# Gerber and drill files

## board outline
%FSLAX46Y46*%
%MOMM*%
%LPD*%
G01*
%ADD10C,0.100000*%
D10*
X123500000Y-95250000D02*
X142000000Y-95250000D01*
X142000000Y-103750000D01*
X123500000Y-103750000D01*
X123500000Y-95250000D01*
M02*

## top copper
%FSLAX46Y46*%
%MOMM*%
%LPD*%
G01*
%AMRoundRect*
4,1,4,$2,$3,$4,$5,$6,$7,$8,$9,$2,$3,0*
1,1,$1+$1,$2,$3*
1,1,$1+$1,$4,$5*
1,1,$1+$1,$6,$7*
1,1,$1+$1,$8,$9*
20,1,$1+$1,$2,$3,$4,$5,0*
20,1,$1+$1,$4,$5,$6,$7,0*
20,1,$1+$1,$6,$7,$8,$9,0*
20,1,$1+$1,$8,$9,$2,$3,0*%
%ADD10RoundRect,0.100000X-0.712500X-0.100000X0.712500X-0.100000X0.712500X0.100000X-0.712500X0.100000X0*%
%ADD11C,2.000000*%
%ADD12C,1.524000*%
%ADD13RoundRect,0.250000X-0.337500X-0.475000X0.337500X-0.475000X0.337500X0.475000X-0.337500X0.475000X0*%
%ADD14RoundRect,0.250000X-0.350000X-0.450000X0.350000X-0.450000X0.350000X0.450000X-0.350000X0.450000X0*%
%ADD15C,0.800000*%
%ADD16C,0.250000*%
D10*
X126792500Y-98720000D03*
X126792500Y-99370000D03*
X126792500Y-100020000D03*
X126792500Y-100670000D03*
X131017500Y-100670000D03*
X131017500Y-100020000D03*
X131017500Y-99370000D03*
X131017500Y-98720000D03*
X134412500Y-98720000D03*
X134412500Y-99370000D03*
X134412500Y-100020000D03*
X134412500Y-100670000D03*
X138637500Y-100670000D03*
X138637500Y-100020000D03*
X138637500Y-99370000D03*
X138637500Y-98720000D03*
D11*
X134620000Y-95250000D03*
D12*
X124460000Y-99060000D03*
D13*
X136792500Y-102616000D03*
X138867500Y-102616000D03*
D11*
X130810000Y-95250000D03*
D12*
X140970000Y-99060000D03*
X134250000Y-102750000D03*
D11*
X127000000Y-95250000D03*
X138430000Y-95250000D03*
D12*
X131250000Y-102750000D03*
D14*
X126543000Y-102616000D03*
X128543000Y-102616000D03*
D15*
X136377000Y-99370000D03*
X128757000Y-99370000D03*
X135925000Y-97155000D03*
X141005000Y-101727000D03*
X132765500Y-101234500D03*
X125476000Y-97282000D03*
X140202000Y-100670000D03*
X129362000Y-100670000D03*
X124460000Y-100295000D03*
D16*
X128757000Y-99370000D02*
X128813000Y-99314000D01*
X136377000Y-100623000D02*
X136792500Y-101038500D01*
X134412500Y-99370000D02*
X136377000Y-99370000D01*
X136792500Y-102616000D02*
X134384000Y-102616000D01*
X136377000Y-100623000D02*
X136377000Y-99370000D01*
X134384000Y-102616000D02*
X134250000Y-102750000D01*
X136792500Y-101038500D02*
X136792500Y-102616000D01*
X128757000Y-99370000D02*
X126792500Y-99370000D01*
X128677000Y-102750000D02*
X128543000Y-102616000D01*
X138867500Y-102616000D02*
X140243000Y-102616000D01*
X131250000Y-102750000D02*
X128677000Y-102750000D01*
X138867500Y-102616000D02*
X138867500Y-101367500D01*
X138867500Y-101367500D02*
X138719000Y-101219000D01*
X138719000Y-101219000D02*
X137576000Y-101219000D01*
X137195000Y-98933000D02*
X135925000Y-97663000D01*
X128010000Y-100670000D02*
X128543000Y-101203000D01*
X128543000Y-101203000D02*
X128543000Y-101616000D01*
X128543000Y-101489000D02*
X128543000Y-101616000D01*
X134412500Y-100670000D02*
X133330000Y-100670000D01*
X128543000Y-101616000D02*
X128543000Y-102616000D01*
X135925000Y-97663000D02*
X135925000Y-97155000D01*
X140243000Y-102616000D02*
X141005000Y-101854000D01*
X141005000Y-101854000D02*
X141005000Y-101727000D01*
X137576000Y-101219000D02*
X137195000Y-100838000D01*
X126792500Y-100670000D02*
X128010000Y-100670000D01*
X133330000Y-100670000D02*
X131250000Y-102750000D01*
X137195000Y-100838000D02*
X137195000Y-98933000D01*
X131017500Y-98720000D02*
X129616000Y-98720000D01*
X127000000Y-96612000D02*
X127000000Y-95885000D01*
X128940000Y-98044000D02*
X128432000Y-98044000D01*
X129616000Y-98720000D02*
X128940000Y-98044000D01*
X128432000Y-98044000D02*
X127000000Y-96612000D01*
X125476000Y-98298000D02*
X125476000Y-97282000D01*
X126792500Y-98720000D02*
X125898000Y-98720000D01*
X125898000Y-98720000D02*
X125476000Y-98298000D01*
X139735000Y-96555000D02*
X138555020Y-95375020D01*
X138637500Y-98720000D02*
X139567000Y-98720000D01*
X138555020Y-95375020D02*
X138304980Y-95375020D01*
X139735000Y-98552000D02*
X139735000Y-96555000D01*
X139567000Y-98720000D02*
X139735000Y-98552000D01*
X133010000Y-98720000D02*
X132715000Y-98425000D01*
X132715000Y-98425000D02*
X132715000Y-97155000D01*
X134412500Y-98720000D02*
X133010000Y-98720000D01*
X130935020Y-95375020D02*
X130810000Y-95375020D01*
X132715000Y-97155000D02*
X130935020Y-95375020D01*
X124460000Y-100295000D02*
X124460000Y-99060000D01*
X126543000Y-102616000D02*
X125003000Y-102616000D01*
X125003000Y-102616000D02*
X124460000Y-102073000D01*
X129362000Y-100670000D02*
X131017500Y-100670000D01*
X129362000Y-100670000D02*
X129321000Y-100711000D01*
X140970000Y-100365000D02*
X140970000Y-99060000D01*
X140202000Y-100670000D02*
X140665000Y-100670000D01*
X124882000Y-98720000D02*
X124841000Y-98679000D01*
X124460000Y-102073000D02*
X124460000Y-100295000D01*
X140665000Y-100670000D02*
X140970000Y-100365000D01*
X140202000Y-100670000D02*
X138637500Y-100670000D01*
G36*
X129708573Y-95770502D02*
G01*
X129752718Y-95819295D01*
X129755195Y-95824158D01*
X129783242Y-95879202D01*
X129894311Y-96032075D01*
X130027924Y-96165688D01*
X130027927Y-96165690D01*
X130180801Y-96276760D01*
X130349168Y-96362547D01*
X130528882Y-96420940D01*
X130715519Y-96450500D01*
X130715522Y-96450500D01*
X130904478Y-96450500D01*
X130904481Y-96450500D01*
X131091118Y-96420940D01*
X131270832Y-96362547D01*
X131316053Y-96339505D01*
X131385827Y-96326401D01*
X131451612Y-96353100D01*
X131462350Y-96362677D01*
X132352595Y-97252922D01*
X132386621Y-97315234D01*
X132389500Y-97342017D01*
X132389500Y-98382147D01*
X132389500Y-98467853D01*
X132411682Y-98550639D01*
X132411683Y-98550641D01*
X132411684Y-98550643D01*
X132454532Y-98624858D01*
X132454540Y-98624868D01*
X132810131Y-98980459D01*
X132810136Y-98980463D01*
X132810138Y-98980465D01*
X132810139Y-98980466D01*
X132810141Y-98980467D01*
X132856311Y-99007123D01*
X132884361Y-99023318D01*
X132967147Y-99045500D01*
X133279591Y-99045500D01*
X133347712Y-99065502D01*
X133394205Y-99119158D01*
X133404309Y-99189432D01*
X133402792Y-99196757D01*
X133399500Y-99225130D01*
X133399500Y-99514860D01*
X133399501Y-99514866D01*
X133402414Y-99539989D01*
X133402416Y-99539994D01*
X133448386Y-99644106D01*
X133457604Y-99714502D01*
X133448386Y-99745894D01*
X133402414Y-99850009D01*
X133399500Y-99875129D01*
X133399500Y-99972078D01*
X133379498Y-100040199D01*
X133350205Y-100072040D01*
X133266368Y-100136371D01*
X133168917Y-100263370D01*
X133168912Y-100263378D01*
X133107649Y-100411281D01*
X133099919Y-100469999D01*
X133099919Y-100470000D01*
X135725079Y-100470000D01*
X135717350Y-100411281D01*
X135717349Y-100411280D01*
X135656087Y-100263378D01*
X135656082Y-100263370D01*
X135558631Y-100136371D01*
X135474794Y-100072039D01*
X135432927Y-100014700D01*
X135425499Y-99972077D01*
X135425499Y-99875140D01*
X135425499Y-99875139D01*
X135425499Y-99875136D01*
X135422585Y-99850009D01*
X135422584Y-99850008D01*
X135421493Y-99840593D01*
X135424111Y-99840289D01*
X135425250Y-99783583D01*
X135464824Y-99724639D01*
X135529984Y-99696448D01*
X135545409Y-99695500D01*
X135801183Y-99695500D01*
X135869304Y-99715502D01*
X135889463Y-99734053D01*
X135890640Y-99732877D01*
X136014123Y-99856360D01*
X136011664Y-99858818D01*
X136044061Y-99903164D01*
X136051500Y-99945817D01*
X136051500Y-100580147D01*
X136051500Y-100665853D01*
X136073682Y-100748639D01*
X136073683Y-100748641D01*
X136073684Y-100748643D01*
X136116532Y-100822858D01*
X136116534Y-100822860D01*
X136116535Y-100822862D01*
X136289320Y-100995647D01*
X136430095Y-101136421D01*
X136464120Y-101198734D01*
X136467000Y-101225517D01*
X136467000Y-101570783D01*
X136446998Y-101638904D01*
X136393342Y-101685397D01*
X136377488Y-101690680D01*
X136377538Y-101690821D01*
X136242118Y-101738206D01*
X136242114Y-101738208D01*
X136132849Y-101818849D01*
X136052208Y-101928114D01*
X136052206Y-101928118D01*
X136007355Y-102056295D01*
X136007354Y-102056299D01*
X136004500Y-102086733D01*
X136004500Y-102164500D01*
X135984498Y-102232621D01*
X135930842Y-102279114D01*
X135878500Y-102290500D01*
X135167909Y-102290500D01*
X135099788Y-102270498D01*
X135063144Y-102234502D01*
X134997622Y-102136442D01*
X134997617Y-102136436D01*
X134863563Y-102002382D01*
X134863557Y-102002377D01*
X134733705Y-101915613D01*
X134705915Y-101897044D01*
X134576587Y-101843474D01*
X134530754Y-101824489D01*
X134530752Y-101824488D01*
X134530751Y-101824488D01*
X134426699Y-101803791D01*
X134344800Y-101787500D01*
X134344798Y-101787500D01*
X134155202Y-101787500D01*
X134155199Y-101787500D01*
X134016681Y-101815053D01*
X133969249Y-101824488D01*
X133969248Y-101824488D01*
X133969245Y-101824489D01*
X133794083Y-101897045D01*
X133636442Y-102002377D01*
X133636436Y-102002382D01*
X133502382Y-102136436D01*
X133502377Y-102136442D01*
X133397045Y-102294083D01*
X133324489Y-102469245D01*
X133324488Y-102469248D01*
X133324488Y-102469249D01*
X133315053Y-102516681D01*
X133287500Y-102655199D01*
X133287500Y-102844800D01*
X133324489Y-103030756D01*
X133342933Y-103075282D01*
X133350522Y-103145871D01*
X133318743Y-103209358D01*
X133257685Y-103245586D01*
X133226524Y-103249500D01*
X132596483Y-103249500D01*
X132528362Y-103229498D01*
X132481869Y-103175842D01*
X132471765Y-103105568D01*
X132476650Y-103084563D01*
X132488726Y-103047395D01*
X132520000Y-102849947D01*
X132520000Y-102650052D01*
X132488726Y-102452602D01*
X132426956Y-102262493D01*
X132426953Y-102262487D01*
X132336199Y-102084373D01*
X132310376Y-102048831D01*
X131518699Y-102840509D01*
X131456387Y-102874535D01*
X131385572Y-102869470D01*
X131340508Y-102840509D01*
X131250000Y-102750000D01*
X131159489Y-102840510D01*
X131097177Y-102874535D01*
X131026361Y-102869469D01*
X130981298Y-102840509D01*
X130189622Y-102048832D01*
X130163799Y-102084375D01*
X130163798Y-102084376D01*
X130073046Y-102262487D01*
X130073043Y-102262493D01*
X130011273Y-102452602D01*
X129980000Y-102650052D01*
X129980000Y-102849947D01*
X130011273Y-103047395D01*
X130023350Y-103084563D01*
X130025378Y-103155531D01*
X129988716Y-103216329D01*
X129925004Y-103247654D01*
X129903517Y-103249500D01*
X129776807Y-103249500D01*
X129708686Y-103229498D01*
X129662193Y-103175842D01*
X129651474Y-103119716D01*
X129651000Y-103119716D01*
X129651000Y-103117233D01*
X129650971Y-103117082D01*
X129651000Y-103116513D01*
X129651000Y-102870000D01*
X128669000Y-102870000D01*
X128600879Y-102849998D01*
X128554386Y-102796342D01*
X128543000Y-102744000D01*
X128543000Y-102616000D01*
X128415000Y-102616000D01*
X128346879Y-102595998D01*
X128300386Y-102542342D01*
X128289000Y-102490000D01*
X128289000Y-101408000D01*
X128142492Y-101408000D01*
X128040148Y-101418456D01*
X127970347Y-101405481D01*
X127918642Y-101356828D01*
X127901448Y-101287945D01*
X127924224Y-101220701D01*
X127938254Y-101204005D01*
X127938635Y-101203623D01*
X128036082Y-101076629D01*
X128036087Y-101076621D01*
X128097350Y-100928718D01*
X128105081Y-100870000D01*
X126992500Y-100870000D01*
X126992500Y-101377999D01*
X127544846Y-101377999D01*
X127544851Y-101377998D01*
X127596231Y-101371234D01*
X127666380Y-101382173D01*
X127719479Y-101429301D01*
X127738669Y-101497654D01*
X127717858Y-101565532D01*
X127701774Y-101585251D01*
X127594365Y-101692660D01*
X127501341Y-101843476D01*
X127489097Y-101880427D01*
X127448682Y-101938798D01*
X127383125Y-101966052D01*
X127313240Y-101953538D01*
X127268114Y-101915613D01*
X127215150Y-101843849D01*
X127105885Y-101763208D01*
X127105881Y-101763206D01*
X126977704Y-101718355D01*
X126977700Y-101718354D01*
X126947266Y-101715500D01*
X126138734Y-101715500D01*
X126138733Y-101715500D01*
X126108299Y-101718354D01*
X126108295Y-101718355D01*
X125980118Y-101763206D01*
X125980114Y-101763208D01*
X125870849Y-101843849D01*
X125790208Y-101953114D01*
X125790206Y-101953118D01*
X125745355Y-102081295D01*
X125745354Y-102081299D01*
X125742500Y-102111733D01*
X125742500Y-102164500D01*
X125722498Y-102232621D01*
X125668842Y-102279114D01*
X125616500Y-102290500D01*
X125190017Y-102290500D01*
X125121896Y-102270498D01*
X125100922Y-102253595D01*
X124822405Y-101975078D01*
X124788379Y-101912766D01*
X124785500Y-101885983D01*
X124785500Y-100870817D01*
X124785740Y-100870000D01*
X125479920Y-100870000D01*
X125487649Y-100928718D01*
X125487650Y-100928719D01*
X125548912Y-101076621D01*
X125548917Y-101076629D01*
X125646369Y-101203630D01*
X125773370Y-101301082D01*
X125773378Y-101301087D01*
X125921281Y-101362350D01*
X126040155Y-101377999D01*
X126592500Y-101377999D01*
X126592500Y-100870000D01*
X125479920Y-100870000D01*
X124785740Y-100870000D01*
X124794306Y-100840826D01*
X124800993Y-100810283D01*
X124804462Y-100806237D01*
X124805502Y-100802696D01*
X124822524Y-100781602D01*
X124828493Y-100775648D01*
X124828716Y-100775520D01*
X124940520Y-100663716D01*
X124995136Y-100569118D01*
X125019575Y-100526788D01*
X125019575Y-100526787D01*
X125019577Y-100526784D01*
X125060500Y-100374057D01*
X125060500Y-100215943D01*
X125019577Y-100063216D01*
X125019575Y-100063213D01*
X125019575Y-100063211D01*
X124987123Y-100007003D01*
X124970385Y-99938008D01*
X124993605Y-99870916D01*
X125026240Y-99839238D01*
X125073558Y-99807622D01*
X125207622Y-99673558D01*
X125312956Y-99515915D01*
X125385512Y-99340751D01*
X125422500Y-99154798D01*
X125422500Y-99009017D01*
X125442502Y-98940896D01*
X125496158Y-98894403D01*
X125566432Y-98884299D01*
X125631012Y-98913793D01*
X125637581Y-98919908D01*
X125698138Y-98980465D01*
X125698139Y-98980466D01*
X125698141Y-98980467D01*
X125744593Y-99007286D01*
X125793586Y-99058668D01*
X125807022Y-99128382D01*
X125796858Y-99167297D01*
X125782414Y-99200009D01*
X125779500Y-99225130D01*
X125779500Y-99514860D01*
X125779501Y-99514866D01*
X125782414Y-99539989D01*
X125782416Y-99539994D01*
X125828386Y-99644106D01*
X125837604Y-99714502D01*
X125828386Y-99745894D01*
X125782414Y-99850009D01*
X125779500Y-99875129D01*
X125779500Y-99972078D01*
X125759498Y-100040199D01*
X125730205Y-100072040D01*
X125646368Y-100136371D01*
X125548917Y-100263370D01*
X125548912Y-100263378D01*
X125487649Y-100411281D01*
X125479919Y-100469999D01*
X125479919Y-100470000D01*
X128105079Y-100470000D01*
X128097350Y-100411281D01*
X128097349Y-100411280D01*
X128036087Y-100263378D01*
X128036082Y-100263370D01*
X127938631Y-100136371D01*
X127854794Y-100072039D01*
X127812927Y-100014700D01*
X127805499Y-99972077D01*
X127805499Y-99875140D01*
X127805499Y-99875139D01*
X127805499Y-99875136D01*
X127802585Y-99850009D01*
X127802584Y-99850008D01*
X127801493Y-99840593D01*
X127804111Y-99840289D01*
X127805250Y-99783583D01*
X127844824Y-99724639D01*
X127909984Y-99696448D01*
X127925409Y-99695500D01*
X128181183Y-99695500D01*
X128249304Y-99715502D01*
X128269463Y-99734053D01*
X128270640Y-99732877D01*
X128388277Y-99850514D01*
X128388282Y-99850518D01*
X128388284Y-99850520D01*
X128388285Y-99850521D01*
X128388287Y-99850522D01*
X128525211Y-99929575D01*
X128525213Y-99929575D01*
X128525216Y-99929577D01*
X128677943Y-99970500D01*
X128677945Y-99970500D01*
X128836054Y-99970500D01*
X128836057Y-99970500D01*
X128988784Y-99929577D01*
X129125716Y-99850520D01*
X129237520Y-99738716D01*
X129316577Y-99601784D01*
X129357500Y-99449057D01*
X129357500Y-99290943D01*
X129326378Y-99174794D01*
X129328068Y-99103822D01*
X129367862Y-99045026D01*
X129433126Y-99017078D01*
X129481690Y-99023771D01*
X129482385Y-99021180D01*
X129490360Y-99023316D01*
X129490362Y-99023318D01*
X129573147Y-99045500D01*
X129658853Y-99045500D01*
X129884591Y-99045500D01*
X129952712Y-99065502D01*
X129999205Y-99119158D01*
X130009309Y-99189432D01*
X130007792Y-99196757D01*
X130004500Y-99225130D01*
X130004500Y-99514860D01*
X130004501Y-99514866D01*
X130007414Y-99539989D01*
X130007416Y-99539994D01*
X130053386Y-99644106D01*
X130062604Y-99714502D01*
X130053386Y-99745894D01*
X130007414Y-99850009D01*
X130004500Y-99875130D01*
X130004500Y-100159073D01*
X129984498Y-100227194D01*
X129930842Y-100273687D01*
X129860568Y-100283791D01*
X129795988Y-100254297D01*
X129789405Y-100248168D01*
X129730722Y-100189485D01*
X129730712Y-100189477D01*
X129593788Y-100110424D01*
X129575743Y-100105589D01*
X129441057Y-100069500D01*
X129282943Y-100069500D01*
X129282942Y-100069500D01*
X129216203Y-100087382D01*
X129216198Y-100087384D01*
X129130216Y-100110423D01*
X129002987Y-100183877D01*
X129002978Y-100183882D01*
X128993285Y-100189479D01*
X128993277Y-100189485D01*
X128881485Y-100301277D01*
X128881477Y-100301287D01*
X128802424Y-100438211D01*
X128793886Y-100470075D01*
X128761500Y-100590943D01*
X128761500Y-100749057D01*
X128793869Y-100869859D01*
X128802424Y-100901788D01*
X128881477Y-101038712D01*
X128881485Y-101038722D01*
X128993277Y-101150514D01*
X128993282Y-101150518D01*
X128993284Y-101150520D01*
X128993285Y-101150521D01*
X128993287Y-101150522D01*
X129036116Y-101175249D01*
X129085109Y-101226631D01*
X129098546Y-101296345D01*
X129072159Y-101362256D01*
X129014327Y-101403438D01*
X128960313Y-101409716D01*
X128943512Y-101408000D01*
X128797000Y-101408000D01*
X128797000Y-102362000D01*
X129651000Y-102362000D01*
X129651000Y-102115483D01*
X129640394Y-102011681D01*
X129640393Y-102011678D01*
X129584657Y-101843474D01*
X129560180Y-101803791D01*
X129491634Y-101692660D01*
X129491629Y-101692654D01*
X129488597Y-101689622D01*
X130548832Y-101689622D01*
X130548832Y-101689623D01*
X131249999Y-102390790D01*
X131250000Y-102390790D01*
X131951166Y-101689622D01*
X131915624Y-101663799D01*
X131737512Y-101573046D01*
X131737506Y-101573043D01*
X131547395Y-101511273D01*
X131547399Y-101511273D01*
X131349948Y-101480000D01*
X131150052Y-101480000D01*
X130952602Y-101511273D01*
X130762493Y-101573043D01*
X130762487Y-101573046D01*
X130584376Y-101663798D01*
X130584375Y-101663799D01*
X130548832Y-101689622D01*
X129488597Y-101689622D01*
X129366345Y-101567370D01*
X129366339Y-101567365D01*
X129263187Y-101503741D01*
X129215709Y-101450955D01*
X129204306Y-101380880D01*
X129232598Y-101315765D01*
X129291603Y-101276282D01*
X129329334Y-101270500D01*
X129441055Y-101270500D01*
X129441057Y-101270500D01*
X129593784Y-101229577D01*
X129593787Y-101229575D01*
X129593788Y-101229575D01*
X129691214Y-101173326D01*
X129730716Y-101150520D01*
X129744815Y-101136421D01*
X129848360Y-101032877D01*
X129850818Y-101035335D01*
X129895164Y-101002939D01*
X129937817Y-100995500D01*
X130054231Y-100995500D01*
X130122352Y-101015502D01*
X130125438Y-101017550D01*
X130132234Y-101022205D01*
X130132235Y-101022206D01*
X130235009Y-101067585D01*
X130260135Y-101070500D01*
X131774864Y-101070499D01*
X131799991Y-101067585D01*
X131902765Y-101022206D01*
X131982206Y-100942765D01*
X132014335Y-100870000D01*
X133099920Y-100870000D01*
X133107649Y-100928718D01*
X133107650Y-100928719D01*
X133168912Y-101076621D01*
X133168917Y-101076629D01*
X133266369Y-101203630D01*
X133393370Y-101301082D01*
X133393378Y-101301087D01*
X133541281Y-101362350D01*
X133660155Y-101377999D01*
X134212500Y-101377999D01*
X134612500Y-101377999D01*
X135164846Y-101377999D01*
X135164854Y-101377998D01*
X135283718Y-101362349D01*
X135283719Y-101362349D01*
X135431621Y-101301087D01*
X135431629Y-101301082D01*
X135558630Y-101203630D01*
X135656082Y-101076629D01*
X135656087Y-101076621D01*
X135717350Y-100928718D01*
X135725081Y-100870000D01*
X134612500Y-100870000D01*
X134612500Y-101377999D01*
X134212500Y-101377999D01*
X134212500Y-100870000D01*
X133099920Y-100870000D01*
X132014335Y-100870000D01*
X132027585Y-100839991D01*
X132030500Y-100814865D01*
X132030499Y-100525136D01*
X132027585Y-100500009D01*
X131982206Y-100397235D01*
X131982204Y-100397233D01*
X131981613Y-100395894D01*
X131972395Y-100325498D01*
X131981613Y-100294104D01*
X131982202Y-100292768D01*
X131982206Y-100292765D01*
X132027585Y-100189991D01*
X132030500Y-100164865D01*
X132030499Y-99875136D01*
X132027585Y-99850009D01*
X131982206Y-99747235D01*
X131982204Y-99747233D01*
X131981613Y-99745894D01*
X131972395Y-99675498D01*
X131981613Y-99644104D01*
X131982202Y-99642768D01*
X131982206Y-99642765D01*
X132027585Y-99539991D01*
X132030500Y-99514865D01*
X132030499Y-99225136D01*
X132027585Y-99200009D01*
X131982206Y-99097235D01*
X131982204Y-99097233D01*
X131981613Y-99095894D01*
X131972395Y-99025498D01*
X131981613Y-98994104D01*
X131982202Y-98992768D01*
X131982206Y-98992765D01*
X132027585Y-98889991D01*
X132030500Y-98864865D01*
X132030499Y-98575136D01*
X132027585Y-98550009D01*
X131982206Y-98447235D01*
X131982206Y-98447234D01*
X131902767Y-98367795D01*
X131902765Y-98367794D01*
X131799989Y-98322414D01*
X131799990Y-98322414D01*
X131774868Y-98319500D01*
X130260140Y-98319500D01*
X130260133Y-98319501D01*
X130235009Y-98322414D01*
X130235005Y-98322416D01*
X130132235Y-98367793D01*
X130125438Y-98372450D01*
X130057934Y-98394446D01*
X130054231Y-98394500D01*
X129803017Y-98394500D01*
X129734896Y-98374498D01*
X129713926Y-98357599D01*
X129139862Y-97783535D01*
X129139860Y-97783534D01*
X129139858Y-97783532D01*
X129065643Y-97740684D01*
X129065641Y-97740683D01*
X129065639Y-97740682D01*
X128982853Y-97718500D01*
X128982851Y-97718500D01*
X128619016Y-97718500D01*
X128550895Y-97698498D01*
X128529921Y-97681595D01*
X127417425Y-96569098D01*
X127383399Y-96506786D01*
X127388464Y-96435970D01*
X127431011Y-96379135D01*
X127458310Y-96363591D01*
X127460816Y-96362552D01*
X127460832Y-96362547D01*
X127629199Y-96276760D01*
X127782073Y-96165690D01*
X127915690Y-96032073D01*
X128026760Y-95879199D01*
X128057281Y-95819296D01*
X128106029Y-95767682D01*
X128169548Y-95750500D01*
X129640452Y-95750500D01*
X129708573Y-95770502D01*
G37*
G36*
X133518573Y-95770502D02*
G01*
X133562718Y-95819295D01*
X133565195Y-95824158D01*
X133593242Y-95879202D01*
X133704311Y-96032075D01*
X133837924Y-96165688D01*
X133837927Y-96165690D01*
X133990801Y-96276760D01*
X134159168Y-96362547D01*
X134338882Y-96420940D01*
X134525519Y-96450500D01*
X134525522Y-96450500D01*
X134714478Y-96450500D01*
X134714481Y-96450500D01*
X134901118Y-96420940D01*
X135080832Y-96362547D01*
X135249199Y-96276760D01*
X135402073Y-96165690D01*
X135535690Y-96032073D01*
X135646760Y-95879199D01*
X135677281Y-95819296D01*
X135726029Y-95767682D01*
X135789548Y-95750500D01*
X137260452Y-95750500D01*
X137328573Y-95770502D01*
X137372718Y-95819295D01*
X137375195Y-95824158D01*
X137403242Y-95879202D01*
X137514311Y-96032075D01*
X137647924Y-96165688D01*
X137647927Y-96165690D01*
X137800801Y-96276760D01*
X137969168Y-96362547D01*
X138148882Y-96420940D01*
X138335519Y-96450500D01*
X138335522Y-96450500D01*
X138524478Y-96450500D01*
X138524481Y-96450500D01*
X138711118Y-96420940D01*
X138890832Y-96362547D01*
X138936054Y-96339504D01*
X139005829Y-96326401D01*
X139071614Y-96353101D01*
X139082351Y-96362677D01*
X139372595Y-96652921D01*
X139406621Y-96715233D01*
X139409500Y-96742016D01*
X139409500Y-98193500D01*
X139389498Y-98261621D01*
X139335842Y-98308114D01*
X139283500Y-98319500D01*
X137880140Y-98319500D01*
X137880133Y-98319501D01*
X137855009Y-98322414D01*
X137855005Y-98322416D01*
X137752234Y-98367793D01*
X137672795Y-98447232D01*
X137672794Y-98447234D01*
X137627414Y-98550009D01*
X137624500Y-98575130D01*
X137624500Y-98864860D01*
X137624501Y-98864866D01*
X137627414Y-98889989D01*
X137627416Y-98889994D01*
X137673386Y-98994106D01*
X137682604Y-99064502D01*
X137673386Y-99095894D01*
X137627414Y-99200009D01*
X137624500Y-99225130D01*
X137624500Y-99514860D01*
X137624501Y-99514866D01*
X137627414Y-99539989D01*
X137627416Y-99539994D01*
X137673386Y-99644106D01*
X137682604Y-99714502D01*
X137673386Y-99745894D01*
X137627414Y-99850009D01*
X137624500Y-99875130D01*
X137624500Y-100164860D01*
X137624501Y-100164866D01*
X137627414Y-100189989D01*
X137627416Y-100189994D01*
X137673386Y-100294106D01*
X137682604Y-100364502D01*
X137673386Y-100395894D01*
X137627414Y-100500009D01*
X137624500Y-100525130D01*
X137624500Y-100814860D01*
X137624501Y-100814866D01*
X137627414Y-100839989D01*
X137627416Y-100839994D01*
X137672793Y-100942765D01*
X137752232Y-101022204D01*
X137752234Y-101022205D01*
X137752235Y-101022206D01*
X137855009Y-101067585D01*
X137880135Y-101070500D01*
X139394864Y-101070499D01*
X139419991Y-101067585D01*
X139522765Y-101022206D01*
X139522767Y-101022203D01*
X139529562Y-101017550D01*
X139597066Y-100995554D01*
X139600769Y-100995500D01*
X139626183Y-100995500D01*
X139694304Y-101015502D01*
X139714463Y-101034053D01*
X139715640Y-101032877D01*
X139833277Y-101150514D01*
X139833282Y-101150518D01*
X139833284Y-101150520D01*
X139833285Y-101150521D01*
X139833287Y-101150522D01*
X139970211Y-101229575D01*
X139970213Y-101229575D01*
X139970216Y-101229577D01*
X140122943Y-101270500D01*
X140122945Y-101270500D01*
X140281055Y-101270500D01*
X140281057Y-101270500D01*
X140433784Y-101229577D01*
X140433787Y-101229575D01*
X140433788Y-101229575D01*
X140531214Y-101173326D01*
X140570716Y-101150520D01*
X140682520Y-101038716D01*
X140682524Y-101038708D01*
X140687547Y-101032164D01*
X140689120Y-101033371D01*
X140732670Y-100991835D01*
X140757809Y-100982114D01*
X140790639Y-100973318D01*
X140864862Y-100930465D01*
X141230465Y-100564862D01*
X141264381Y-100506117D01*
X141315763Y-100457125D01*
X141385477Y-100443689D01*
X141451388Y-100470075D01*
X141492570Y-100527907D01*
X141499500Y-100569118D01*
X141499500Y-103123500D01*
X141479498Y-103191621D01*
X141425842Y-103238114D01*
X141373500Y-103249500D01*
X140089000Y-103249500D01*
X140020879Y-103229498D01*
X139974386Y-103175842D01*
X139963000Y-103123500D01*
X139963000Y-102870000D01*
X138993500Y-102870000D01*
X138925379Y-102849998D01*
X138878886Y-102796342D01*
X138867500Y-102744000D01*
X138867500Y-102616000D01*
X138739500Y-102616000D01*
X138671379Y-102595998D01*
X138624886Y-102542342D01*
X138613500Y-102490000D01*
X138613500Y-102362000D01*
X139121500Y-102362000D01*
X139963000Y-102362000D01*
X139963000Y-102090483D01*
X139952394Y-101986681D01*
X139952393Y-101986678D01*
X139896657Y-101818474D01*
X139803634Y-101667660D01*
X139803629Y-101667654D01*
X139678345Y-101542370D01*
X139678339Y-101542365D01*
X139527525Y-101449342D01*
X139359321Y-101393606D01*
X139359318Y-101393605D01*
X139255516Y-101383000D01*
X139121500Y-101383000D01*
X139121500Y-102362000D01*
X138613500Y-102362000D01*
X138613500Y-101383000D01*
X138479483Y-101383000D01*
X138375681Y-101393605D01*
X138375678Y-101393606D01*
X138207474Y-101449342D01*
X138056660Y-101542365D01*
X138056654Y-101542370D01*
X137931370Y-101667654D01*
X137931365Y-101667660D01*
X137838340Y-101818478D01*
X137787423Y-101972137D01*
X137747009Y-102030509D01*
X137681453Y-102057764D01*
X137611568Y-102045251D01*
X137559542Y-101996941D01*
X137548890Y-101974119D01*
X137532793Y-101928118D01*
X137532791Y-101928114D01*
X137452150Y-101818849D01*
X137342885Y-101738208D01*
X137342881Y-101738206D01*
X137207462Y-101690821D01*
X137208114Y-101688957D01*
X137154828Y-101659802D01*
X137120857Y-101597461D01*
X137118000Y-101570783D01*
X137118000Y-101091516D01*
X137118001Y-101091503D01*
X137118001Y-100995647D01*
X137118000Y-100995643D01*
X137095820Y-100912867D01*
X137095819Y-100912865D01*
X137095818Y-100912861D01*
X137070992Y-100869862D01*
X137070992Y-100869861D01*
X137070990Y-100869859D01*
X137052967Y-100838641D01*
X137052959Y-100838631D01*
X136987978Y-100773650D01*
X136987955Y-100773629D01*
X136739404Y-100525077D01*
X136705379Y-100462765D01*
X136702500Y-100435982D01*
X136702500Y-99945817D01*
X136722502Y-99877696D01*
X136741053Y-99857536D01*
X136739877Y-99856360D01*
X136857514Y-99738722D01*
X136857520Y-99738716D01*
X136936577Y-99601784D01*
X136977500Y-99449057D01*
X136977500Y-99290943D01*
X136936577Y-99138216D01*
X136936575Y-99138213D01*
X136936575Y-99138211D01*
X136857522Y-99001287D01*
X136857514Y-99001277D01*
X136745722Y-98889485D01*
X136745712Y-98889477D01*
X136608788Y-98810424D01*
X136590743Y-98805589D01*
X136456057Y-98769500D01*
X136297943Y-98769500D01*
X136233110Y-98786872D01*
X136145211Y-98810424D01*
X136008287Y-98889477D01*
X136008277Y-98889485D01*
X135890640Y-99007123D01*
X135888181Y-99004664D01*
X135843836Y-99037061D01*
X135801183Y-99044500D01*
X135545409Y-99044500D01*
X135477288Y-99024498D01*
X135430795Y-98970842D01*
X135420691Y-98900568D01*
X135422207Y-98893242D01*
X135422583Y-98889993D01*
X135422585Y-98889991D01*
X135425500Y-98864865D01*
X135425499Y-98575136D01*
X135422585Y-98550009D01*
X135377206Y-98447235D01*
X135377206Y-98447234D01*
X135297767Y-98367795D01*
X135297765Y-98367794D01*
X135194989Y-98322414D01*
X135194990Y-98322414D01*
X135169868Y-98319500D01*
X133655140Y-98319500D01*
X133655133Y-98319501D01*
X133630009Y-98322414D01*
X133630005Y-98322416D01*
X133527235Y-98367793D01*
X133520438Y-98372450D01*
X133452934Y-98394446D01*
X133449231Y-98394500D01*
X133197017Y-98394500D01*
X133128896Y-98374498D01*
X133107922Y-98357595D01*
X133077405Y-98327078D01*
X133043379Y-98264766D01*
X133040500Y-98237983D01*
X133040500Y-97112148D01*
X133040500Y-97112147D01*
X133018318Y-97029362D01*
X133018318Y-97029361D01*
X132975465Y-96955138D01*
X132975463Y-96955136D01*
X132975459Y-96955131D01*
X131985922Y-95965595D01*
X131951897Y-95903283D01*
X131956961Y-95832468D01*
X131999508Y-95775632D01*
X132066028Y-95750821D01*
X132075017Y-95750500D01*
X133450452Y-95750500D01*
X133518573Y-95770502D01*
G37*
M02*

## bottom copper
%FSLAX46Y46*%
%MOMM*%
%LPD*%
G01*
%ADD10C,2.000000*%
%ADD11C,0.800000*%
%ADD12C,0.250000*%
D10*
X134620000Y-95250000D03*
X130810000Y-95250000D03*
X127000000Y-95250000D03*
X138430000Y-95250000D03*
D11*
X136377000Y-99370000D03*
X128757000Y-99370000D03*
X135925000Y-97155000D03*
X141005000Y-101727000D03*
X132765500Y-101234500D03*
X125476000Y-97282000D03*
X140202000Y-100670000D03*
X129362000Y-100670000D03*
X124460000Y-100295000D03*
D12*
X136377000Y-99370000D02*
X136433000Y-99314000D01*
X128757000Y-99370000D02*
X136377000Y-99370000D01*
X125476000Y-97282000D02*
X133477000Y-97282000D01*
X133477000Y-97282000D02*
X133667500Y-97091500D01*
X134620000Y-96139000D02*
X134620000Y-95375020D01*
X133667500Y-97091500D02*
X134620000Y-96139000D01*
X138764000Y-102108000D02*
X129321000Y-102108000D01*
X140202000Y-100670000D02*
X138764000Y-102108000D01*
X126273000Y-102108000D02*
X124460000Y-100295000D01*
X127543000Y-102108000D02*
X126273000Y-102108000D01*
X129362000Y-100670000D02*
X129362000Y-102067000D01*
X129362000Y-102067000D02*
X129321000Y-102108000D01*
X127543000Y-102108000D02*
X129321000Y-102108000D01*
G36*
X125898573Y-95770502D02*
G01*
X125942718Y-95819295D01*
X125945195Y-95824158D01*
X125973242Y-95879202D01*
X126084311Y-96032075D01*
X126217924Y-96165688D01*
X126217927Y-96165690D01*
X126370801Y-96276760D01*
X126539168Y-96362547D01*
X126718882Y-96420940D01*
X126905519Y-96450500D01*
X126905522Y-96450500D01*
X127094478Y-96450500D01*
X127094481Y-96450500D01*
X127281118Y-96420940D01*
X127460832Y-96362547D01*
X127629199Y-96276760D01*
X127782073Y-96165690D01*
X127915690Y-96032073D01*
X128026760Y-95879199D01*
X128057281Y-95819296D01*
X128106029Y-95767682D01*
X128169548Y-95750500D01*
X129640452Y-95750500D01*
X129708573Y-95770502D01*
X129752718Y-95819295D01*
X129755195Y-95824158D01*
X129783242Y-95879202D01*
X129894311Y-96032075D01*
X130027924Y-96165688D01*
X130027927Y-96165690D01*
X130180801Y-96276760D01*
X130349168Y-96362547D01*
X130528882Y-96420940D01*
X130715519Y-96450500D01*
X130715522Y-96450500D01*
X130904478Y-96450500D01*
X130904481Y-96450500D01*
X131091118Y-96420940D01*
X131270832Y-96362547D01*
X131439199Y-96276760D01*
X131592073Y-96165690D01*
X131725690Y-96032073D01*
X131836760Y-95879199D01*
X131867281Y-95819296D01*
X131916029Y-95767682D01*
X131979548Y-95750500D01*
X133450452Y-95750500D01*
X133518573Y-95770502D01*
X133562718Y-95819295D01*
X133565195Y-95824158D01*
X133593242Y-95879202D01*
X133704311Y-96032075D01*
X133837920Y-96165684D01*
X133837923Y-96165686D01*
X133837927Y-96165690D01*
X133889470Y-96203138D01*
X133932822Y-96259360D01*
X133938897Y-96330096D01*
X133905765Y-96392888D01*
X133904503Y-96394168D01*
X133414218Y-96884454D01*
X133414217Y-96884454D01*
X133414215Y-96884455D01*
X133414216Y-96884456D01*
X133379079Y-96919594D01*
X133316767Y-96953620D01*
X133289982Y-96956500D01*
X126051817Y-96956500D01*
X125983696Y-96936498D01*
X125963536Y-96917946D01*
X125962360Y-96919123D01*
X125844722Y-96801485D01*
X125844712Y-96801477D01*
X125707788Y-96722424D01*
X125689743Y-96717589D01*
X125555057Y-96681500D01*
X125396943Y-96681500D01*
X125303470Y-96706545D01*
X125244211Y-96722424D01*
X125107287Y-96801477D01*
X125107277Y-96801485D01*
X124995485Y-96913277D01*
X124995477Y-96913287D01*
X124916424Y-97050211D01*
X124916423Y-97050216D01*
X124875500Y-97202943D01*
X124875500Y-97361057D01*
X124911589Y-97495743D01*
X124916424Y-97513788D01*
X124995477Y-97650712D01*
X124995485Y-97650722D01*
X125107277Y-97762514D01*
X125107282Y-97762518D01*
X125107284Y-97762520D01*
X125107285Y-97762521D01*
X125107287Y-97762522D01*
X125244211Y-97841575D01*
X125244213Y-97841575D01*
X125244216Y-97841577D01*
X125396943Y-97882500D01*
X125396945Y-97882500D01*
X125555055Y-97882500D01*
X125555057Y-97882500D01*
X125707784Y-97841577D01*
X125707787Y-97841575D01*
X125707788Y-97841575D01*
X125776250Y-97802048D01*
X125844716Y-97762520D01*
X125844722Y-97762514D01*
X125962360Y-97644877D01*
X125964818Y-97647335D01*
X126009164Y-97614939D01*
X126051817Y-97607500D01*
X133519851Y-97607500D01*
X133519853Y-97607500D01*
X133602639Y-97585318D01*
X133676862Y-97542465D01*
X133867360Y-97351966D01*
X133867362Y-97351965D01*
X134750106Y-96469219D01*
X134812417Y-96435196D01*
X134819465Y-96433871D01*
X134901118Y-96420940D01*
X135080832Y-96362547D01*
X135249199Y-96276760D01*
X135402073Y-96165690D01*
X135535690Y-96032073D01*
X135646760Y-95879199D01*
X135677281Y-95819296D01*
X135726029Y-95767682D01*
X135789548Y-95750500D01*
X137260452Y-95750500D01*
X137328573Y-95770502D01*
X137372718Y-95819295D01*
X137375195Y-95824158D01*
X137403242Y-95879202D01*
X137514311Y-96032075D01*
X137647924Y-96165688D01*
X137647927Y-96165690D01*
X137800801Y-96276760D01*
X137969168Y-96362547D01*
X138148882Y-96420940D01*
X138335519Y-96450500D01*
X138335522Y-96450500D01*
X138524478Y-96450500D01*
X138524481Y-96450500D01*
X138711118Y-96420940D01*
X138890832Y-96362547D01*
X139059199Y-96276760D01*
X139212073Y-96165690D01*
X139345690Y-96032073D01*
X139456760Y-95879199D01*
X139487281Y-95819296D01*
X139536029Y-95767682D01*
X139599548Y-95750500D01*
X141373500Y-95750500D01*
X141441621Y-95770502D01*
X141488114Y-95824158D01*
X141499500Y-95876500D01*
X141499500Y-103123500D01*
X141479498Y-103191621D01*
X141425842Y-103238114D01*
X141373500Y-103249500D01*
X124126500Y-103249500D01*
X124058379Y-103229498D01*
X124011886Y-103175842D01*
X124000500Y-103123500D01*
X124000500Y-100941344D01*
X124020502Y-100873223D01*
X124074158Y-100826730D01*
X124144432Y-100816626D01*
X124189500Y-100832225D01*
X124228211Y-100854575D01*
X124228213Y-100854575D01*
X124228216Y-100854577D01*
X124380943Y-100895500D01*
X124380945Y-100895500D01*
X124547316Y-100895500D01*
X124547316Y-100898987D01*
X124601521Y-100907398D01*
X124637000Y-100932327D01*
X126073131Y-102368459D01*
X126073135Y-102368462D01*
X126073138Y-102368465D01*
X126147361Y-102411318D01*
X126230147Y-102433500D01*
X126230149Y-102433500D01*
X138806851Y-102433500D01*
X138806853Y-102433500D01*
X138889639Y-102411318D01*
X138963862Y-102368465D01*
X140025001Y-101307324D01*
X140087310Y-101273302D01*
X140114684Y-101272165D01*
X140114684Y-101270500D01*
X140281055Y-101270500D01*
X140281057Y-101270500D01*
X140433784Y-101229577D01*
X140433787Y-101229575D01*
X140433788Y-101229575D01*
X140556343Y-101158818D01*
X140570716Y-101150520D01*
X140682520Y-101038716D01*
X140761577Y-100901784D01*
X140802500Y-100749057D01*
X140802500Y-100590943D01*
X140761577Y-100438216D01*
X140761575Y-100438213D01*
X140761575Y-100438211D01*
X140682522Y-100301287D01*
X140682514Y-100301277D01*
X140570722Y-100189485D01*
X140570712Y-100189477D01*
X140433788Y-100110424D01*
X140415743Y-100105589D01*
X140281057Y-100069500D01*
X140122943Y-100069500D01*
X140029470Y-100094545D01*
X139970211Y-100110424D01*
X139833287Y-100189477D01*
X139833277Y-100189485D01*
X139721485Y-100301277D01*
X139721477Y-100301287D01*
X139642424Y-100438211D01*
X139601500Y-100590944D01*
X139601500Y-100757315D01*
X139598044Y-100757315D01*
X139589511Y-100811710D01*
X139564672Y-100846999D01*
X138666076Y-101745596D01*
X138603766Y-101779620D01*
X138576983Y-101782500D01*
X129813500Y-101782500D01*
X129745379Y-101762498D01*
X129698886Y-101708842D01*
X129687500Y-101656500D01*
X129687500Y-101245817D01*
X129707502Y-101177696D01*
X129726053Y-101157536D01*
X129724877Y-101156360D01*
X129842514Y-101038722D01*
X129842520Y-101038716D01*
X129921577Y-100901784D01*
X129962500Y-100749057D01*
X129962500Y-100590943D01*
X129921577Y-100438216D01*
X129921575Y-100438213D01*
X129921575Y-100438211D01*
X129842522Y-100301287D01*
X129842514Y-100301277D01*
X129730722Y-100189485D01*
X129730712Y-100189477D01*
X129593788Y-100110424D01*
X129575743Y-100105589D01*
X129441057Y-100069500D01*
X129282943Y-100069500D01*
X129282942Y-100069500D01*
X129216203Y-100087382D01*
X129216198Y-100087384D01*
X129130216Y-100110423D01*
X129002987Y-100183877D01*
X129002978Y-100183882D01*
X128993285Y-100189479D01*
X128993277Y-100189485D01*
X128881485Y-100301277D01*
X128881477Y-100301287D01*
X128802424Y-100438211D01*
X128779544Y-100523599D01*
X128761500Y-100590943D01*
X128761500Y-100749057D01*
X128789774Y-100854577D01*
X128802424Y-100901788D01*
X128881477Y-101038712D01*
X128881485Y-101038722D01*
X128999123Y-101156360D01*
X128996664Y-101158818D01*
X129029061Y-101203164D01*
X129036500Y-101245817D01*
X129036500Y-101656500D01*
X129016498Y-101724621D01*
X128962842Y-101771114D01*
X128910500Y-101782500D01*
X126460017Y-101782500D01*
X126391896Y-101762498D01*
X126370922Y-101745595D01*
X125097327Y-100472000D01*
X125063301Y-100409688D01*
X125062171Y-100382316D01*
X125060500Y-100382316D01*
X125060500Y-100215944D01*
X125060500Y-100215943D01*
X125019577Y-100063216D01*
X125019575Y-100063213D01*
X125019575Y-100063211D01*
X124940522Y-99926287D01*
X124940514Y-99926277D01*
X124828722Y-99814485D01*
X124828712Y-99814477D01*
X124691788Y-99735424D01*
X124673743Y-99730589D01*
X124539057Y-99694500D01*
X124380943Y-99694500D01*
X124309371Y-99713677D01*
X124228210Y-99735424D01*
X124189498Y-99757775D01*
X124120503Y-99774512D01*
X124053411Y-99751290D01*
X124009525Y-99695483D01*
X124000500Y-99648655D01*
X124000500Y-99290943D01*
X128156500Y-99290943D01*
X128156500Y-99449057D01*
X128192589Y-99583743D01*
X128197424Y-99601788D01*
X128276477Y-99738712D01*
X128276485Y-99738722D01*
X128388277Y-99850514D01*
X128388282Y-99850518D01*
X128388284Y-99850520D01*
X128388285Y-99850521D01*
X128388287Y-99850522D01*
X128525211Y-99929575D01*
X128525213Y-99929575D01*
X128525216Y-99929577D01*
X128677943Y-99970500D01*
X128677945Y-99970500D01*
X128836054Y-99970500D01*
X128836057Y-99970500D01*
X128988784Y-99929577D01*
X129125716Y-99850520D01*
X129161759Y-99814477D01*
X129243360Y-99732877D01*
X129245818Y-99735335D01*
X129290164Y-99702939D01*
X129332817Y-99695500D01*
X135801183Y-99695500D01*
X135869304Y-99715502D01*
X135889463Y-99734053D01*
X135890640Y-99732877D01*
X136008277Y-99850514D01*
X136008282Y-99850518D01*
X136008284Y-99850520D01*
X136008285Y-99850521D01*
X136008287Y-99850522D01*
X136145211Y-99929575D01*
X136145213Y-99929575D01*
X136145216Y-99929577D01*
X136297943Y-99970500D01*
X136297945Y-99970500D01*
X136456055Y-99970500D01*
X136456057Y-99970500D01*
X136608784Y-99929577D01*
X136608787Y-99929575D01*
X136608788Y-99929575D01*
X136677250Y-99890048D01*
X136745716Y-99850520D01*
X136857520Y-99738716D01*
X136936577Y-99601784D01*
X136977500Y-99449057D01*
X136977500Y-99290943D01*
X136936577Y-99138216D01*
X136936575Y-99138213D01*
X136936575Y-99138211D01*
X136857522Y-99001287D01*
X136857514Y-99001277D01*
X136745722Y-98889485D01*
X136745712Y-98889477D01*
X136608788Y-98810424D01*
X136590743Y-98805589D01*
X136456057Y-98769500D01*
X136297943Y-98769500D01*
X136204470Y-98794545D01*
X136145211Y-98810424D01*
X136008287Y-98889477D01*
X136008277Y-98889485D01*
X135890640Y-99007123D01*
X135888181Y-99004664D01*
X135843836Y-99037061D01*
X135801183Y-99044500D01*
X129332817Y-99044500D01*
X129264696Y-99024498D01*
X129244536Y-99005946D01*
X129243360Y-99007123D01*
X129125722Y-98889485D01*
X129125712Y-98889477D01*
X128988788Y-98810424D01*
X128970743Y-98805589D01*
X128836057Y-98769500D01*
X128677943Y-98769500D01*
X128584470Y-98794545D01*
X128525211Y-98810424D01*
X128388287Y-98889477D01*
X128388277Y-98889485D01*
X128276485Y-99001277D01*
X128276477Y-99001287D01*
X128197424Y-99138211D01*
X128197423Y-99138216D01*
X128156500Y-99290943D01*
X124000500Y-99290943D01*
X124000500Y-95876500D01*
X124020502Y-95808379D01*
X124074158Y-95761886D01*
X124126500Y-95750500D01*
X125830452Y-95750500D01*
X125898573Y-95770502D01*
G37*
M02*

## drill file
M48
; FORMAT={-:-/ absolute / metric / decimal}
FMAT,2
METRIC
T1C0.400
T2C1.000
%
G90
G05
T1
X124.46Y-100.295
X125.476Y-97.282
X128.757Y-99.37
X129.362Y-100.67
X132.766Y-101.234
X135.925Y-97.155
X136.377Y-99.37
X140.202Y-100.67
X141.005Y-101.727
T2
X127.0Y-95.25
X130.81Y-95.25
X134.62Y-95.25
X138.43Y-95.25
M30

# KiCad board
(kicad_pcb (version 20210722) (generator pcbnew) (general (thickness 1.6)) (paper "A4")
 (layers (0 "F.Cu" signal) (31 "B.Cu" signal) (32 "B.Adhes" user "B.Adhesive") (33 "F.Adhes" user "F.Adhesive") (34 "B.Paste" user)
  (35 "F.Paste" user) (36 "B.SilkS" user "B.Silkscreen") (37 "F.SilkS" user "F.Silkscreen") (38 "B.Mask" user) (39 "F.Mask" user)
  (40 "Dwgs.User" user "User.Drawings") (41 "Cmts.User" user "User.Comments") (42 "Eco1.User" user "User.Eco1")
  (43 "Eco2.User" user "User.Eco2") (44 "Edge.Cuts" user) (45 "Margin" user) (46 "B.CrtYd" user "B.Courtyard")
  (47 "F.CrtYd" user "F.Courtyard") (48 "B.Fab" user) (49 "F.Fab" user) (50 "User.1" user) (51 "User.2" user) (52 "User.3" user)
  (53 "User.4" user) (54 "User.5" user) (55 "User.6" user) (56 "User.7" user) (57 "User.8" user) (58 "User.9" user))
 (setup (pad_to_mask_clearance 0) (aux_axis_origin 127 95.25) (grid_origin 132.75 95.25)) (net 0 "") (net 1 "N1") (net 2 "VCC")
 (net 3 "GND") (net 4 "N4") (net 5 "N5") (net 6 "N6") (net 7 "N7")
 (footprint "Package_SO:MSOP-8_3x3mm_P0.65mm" (layer "F.Cu") (at 128.905 99.695)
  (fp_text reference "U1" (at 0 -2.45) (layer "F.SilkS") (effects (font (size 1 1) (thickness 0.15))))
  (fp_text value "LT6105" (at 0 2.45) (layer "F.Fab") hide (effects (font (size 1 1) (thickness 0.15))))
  (pad "1" smd roundrect locked (at -2.1125 -0.975) (size 1.625 0.4) (layers "F.Cu" "F.Paste" "F.Mask") (roundrect_rratio 0.25) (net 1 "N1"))
  (pad "2" smd roundrect locked (at -2.1125 -0.325) (size 1.625 0.4) (layers "F.Cu" "F.Paste" "F.Mask") (roundrect_rratio 0.25)
   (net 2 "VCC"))
  (pad "3" smd roundrect locked (at -2.1125 0.325) (size 1.625 0.4) (layers "F.Cu" "F.Paste" "F.Mask") (roundrect_rratio 0.25))
  (pad "4" smd roundrect locked (at -2.1125 0.975) (size 1.625 0.4) (layers "F.Cu" "F.Paste" "F.Mask") (roundrect_rratio 0.25) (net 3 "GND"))
  (pad "5" smd roundrect locked (at 2.1125 0.975) (size 1.625 0.4) (layers "F.Cu" "F.Paste" "F.Mask") (roundrect_rratio 0.25) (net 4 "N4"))
  (pad "6" smd roundrect locked (at 2.1125 0.325) (size 1.625 0.4) (layers "F.Cu" "F.Paste" "F.Mask") (roundrect_rratio 0.25))
  (pad "7" smd roundrect locked (at 2.1125 -0.325) (size 1.625 0.4) (layers "F.Cu" "F.Paste" "F.Mask") (roundrect_rratio 0.25))
  (pad "8" smd roundrect locked (at 2.1125 -0.975) (size 1.625 0.4) (layers "F.Cu" "F.Paste" "F.Mask") (roundrect_rratio 0.25) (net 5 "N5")))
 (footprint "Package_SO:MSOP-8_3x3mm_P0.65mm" (layer "F.Cu") (at 136.525 99.695)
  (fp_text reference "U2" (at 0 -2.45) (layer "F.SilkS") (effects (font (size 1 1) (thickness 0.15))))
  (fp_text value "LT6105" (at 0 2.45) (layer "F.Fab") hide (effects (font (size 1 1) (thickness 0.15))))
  (pad "1" smd roundrect locked (at -2.1125 -0.975) (size 1.625 0.4) (layers "F.Cu" "F.Paste" "F.Mask") (roundrect_rratio 0.25) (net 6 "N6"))
  (pad "2" smd roundrect locked (at -2.1125 -0.325) (size 1.625 0.4) (layers "F.Cu" "F.Paste" "F.Mask") (roundrect_rratio 0.25)
   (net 2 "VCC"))
  (pad "3" smd roundrect locked (at -2.1125 0.325) (size 1.625 0.4) (layers "F.Cu" "F.Paste" "F.Mask") (roundrect_rratio 0.25))
  (pad "4" smd roundrect locked (at -2.1125 0.975) (size 1.625 0.4) (layers "F.Cu" "F.Paste" "F.Mask") (roundrect_rratio 0.25) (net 3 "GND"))
  (pad "5" smd roundrect locked (at 2.1125 0.975) (size 1.625 0.4) (layers "F.Cu" "F.Paste" "F.Mask") (roundrect_rratio 0.25) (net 4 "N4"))
  (pad "6" smd roundrect locked (at 2.1125 0.325) (size 1.625 0.4) (layers "F.Cu" "F.Paste" "F.Mask") (roundrect_rratio 0.25))
  (pad "7" smd roundrect locked (at 2.1125 -0.325) (size 1.625 0.4) (layers "F.Cu" "F.Paste" "F.Mask") (roundrect_rratio 0.25))
  (pad "8" smd roundrect locked (at 2.1125 -0.975) (size 1.625 0.4) (layers "F.Cu" "F.Paste" "F.Mask") (roundrect_rratio 0.25) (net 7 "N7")))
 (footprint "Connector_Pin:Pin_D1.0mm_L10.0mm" (layer "F.Cu") (at 134.62 95.25)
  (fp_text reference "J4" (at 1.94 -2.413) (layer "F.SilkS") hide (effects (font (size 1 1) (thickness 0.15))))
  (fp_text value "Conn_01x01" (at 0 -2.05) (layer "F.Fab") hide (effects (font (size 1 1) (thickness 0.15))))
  (pad "1" thru_hole circle locked (at 0 0) (size 2 2) (drill 1) (layers *.Cu *.Mask) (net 1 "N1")))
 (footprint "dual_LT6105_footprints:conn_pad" (layer "F.Cu") (at 124.46 99.06)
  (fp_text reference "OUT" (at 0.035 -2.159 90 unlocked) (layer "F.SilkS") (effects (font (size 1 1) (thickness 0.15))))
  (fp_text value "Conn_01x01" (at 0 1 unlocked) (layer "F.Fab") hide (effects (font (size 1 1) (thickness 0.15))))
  (pad "1" smd circle (at 0 0) (size 1.524 1.524) (layers "F.Cu" "F.Paste" "F.Mask") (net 4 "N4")))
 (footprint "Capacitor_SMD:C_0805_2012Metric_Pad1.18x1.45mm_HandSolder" (layer "F.Cu") (at 137.83 102.616)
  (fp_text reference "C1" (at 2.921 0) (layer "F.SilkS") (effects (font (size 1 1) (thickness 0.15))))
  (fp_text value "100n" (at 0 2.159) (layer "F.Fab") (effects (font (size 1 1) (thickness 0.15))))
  (pad "1" smd roundrect locked (at -1.0375 0) (size 1.175 1.45) (layers "F.Cu" "F.Paste" "F.Mask") (roundrect_rratio 0.2127659574)
   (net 2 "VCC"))
  (pad "2" smd roundrect locked (at 1.0375 0) (size 1.175 1.45) (layers "F.Cu" "F.Paste" "F.Mask") (roundrect_rratio 0.2127659574)
   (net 3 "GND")))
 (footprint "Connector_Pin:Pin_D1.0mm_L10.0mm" (layer "F.Cu") (at 130.81 95.25)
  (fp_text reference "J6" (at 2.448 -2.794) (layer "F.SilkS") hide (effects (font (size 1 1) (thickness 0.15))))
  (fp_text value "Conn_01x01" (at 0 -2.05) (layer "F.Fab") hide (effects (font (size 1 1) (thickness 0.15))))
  (pad "1" thru_hole circle locked (at 0 0) (size 2 2) (drill 1) (layers *.Cu *.Mask) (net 6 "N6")))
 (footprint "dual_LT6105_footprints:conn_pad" (layer "F.Cu") (at 140.97 99.06)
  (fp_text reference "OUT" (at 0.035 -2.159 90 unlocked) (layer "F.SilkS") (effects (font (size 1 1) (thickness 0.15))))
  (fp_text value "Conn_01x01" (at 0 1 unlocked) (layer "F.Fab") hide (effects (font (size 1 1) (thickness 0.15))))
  (pad "1" smd circle (at 0 0) (size 1.524 1.524) (layers "F.Cu" "F.Paste" "F.Mask") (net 4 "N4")))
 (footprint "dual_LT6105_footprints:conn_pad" (layer "F.Cu") (at 134.25 102.75)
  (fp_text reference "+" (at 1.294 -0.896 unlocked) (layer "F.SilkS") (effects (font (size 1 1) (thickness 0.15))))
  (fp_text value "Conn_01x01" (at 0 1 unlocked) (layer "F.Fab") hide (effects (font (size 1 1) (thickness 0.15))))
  (pad "1" smd circle (at 0 0) (size 1.524 1.524) (layers "F.Cu" "F.Paste" "F.Mask") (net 2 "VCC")))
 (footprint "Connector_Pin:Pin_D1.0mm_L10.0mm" (layer "F.Cu") (at 127 95.25)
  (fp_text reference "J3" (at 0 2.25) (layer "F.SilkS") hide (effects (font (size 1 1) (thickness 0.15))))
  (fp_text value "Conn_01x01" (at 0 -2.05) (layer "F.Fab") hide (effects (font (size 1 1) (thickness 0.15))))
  (pad "1" thru_hole circle locked (at 0 0) (size 2 2) (drill 1) (layers *.Cu *.Mask) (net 5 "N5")))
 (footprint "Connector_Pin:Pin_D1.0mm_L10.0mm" (layer "F.Cu") (at 138.43 95.25)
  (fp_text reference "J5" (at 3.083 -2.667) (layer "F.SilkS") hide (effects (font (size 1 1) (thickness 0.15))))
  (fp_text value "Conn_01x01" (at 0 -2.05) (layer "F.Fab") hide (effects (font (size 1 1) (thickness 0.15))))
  (pad "1" thru_hole circle locked (at 0 0) (size 2 2) (drill 1) (layers *.Cu *.Mask) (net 7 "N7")))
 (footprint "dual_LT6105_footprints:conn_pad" (layer "F.Cu") (at 131.25 102.75)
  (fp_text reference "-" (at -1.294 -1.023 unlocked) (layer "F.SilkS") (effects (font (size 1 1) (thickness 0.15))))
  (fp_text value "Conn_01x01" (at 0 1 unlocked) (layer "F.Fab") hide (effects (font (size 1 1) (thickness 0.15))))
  (pad "1" smd circle (at 0 0) (size 1.524 1.524) (layers "F.Cu" "F.Paste" "F.Mask") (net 3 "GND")))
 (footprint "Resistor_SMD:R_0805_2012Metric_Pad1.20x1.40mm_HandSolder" (layer "F.Cu") (at 127.543 102.616)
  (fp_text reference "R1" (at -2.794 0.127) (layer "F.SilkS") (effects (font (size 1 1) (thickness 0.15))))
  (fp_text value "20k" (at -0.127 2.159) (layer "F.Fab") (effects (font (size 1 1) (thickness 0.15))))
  (pad "1" smd roundrect locked (at -1 0) (size 1.2 1.4) (layers "F.Cu" "F.Paste" "F.Mask") (roundrect_rratio 0.2083333333) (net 4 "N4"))
  (pad "2" smd roundrect locked (at 1 0) (size 1.2 1.4) (layers "F.Cu" "F.Paste" "F.Mask") (roundrect_rratio 0.2083333333) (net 3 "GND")))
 (gr_rect (start 123.5 103.75) (end 142 95.25) (layer "Edge.Cuts") (width 0.1) (fill none))
 (segment (start 128.757 99.37) (end 128.813 99.314) (width 0.25) (layer "F.Cu") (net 2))
 (segment (start 136.377 100.623) (end 136.7925 101.0385) (width 0.25) (layer "F.Cu") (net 2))
 (segment (start 134.4125 99.37) (end 136.377 99.37) (width 0.25) (layer "F.Cu") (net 2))
 (segment (start 136.7925 102.616) (end 134.384 102.616) (width 0.25) (layer "F.Cu") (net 2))
 (segment (start 136.377 100.623) (end 136.377 99.37) (width 0.25) (layer "F.Cu") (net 2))
 (segment (start 134.384 102.616) (end 134.25 102.75) (width 0.25) (layer "F.Cu") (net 2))
 (segment (start 136.7925 101.0385) (end 136.7925 102.616) (width 0.25) (layer "F.Cu") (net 2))
 (segment (start 128.757 99.37) (end 126.7925 99.37) (width 0.25) (layer "F.Cu") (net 2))
 (via (at 136.377 99.37) (size 0.8) (drill 0.4) (layers "F.Cu" "B.Cu") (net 2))
 (via (at 128.757 99.37) (size 0.8) (drill 0.4) (layers "F.Cu" "B.Cu") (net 2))
 (segment (start 136.377 99.37) (end 136.433 99.314) (width 0.25) (layer "B.Cu") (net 2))
 (segment (start 128.757 99.37) (end 136.377 99.37) (width 0.25) (layer "B.Cu") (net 2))
 (segment (start 128.677 102.75) (end 128.543 102.616) (width 0.25) (layer "F.Cu") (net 3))
 (segment (start 138.8675 102.616) (end 140.243 102.616) (width 0.25) (layer "F.Cu") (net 3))
 (segment (start 131.25 102.75) (end 128.677 102.75) (width 0.25) (layer "F.Cu") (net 3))
 (segment (start 138.8675 102.616) (end 138.8675 101.3675) (width 0.25) (layer "F.Cu") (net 3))
 (segment (start 138.8675 101.3675) (end 138.719 101.219) (width 0.25) (layer "F.Cu") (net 3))
 (segment (start 138.719 101.219) (end 137.576 101.219) (width 0.25) (layer "F.Cu") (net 3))
 (segment (start 137.195 98.933) (end 135.925 97.663) (width 0.25) (layer "F.Cu") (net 3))
 (segment (start 128.01 100.67) (end 128.543 101.203) (width 0.25) (layer "F.Cu") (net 3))
 (segment (start 128.543 101.203) (end 128.543 101.616) (width 0.25) (layer "F.Cu") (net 3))
 (segment (start 128.543 101.489) (end 128.543 101.616) (width 0.25) (layer "F.Cu") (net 3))
 (segment (start 134.4125 100.67) (end 133.33 100.67) (width 0.25) (layer "F.Cu") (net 3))
 (segment (start 128.543 101.616) (end 128.543 102.616) (width 0.25) (layer "F.Cu") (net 3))
 (segment (start 135.925 97.663) (end 135.925 97.155) (width 0.25) (layer "F.Cu") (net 3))
 (segment (start 140.243 102.616) (end 141.005 101.854) (width 0.25) (layer "F.Cu") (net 3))
 (segment (start 141.005 101.854) (end 141.005 101.727) (width 0.25) (layer "F.Cu") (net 3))
 (segment (start 137.576 101.219) (end 137.195 100.838) (width 0.25) (layer "F.Cu") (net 3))
 (segment (start 126.7925 100.67) (end 128.01 100.67) (width 0.25) (layer "F.Cu") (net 3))
 (segment (start 133.33 100.67) (end 131.25 102.75) (width 0.25) (layer "F.Cu") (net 3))
 (segment (start 137.195 100.838) (end 137.195 98.933) (width 0.25) (layer "F.Cu") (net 3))
 (via (at 135.925 97.155) (size 0.8) (drill 0.4) (layers "F.Cu" "B.Cu") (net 3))
 (via (at 141.005 101.727) (size 0.8) (drill 0.4) (layers "F.Cu" "B.Cu") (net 3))
 (via (at 132.7655 101.2345) (size 0.8) (drill 0.4) (layers "F.Cu" "B.Cu") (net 3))
 (segment (start 131.0175 98.72) (end 129.616 98.72) (width 0.25) (layer "F.Cu") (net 5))
 (segment (start 127 96.612) (end 127 95.885) (width 0.25) (layer "F.Cu") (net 5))
 (segment (start 128.94 98.044) (end 128.432 98.044) (width 0.25) (layer "F.Cu") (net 5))
 (segment (start 129.616 98.72) (end 128.94 98.044) (width 0.25) (layer "F.Cu") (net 5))
 (segment (start 128.432 98.044) (end 127 96.612) (width 0.25) (layer "F.Cu") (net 5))
 (segment (start 125.476 98.298) (end 125.476 97.282) (width 0.25) (layer "F.Cu") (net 1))
 (segment (start 126.7925 98.72) (end 125.898 98.72) (width 0.25) (layer "F.Cu") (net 1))
 (segment (start 125.898 98.72) (end 125.476 98.298) (width 0.25) (layer "F.Cu") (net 1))
 (via (at 125.476 97.282) (size 0.8) (drill 0.4) (layers "F.Cu" "B.Cu") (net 1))
 (segment (start 125.476 97.282) (end 133.477 97.282) (width 0.25) (layer "B.Cu") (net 1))
 (segment (start 133.477 97.282) (end 133.6675 97.0915) (width 0.25) (layer "B.Cu") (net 1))
 (segment (start 134.62 96.139) (end 134.62 95.37502) (width 0.25) (layer "B.Cu") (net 1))
 (segment (start 133.6675 97.0915) (end 134.62 96.139) (width 0.25) (layer "B.Cu") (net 1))
 (segment (start 139.735 96.555) (end 138.55502 95.37502) (width 0.25) (layer "F.Cu") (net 7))
 (segment (start 138.6375 98.72) (end 139.567 98.72) (width 0.25) (layer "F.Cu") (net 7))
 (segment (start 138.55502 95.37502) (end 138.30498 95.37502) (width 0.25) (layer "F.Cu") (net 7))
 (segment (start 139.735 98.552) (end 139.735 96.555) (width 0.25) (layer "F.Cu") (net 7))
 (segment (start 139.567 98.72) (end 139.735 98.552) (width 0.25) (layer "F.Cu") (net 7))
 (segment (start 133.01 98.72) (end 132.715 98.425) (width 0.25) (layer "F.Cu") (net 6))
 (segment (start 132.715 98.425) (end 132.715 97.155) (width 0.25) (layer "F.Cu") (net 6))
 (segment (start 134.4125 98.72) (end 133.01 98.72) (width 0.25) (layer "F.Cu") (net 6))
 (segment (start 130.93502 95.37502) (end 130.81 95.37502) (width 0.25) (layer "F.Cu") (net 6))
 (segment (start 132.715 97.155) (end 130.93502 95.37502) (width 0.25) (layer "F.Cu") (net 6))
 (segment (start 124.46 100.295) (end 124.46 99.06) (width 0.25) (layer "F.Cu") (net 4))
 (segment (start 126.543 102.616) (end 125.003 102.616) (width 0.25) (layer "F.Cu") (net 4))
 (segment (start 125.003 102.616) (end 124.46 102.073) (width 0.25) (layer "F.Cu") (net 4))
 (segment (start 129.362 100.67) (end 131.0175 100.67) (width 0.25) (layer "F.Cu") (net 4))
 (segment (start 129.362 100.67) (end 129.321 100.711) (width 0.25) (layer "F.Cu") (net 4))
 (segment (start 140.97 100.365) (end 140.97 99.06) (width 0.25) (layer "F.Cu") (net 4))
 (segment (start 140.202 100.67) (end 140.665 100.67) (width 0.25) (layer "F.Cu") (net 4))
 (segment (start 124.882 98.72) (end 124.841 98.679) (width 0.25) (layer "F.Cu") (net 4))
 (segment (start 124.46 102.073) (end 124.46 100.295) (width 0.25) (layer "F.Cu") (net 4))
 (segment (start 140.665 100.67) (end 140.97 100.365) (width 0.25) (layer "F.Cu") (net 4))
 (segment (start 140.202 100.67) (end 138.6375 100.67) (width 0.25) (layer "F.Cu") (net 4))
 (via (at 140.202 100.67) (size 0.8) (drill 0.4) (layers "F.Cu" "B.Cu") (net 4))
 (via (at 129.362 100.67) (size 0.8) (drill 0.4) (layers "F.Cu" "B.Cu") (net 4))
 (via (at 124.46 100.295) (size 0.8) (drill 0.4) (layers "F.Cu" "B.Cu") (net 4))
 (segment (start 138.764 102.108) (end 129.321 102.108) (width 0.25) (layer "B.Cu") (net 4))
 (segment (start 140.202 100.67) (end 138.764 102.108) (width 0.25) (layer "B.Cu") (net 4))
 (segment (start 126.273 102.108) (end 124.46 100.295) (width 0.25) (layer "B.Cu") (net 4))
 (segment (start 127.543 102.108) (end 126.273 102.108) (width 0.25) (layer "B.Cu") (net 4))
 (segment (start 129.362 100.67) (end 129.362 102.067) (width 0.25) (layer "B.Cu") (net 4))
 (segment (start 129.362 102.067) (end 129.321 102.108) (width 0.25) (layer "B.Cu") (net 4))
 (segment (start 127.543 102.108) (end 129.321 102.108) (width 0.25) (layer "B.Cu") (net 4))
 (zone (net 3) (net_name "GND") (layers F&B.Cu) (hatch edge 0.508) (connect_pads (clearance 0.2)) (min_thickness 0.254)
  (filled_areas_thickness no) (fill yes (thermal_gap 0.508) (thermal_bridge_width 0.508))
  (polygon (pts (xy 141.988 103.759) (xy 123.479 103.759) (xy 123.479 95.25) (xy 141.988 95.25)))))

